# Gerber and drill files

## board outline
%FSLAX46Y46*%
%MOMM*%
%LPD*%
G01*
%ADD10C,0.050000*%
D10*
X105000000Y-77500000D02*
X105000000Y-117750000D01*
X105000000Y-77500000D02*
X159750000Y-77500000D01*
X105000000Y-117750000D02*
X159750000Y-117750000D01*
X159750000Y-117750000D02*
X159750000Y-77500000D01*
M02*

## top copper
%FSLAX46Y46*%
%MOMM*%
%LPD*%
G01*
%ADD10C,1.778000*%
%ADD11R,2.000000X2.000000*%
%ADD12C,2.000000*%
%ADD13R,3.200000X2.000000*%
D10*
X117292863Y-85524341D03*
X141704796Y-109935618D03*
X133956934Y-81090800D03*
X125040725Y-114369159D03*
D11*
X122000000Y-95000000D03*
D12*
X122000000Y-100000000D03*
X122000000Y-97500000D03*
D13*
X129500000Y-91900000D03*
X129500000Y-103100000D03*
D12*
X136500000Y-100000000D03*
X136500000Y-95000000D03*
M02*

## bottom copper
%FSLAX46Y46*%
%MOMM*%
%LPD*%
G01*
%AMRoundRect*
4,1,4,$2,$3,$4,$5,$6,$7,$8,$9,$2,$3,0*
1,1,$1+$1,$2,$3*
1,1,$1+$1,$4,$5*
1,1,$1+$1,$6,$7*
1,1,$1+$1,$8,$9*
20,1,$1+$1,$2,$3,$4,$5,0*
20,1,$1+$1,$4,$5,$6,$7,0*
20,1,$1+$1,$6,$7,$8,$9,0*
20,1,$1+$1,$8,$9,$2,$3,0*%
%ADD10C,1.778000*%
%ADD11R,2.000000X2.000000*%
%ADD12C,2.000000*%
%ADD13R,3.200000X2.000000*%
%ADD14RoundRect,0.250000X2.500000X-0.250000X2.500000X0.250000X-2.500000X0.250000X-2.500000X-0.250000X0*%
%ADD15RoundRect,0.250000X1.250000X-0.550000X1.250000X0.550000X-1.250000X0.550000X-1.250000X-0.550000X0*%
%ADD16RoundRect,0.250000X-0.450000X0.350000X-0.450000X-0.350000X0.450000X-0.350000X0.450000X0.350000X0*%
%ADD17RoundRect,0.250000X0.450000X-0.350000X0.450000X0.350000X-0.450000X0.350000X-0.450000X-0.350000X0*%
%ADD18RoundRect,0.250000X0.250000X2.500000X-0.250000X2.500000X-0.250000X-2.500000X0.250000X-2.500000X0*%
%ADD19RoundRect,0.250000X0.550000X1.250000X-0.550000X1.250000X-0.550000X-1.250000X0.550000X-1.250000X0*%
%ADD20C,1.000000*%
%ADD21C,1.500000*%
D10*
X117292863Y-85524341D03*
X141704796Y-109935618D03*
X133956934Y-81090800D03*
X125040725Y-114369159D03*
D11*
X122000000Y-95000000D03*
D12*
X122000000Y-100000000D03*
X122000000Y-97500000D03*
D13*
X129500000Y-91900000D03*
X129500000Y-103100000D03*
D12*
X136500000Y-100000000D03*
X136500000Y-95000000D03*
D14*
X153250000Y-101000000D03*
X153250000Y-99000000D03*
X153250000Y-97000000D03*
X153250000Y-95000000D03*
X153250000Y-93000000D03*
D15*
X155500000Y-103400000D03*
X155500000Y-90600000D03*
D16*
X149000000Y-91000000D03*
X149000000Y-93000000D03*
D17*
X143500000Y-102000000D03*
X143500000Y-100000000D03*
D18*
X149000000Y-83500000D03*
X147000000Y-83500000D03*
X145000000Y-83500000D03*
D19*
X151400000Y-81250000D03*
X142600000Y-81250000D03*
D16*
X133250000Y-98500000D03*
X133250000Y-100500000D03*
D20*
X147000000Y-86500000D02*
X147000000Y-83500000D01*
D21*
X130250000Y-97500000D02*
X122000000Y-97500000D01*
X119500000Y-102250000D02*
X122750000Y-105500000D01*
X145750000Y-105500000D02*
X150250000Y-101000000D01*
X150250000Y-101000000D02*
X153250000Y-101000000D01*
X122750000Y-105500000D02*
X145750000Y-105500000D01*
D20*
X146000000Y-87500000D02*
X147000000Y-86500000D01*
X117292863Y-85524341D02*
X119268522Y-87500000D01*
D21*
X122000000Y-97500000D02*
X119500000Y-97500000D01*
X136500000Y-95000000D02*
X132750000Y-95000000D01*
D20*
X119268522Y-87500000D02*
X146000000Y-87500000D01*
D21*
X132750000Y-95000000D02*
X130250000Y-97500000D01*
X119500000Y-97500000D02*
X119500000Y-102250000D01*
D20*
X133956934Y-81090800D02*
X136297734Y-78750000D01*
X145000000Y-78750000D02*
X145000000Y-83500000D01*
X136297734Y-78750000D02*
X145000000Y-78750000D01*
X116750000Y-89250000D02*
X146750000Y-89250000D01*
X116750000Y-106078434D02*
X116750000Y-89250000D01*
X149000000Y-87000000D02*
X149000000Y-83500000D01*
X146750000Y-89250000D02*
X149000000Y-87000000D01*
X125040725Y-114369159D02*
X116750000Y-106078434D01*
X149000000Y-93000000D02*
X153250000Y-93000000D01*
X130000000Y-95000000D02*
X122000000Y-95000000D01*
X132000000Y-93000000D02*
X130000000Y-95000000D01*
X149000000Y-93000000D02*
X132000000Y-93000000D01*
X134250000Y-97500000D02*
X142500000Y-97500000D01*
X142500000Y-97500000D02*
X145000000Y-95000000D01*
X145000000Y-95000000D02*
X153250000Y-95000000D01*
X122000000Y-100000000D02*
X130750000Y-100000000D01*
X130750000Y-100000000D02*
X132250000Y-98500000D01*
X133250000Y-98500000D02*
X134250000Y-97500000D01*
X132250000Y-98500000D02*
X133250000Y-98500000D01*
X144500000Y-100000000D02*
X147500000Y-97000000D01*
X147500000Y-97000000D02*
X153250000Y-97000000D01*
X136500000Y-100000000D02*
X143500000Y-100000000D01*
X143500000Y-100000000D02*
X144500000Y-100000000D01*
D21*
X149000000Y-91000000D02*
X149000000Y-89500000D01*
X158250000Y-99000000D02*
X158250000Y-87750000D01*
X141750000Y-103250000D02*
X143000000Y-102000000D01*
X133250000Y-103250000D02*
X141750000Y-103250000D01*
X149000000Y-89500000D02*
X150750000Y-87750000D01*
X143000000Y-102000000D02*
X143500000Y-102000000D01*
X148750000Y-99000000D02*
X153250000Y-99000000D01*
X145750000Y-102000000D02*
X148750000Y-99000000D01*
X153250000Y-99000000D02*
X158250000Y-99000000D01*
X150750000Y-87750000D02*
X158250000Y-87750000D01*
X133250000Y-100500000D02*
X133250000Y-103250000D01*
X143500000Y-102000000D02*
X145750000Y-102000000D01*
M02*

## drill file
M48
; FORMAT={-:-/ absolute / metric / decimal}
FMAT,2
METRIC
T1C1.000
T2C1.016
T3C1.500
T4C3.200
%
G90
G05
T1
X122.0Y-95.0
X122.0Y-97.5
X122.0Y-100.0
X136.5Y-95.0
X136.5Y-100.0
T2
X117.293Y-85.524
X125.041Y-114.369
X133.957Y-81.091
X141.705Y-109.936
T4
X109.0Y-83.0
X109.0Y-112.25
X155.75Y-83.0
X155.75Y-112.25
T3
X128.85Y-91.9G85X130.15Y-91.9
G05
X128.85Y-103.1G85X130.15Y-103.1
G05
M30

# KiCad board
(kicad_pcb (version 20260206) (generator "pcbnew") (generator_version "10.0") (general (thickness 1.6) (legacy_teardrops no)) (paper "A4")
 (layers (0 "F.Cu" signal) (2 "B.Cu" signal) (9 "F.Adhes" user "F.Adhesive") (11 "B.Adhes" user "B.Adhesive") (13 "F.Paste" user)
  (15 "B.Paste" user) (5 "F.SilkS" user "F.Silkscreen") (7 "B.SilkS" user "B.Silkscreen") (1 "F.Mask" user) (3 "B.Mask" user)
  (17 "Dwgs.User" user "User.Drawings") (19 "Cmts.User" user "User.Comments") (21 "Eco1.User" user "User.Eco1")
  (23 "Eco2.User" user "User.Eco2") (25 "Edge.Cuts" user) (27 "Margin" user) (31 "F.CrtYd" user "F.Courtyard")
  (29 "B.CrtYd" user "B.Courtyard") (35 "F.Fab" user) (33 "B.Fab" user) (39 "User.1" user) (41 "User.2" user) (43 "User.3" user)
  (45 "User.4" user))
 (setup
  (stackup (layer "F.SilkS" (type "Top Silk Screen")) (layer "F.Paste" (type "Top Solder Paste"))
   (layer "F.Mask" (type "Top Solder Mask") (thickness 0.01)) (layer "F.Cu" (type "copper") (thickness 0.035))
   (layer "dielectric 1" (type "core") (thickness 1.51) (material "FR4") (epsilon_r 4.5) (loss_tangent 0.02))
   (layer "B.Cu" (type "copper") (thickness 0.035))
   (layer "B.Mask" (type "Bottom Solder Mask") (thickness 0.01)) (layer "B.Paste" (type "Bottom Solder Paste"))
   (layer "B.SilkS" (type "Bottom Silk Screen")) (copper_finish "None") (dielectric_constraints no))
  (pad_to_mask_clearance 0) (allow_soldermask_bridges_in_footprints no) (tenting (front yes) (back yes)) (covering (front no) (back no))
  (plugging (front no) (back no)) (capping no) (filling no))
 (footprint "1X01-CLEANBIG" (layer "F.Cu") (at 117.292863 85.524341 180)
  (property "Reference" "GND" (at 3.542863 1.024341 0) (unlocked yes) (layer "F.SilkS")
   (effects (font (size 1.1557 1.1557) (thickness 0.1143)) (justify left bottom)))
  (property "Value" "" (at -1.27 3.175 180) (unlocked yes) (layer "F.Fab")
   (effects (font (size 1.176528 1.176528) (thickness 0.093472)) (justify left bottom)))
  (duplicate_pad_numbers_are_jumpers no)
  (pad "1" thru_hole circle (at 0 0 180) (size 1.778 1.778) (drill 1.016) (layers "*.Cu" "*.Mask") (remove_unused_layers no) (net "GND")
   (solder_mask_margin 0.1016) (thermal_bridge_angle 0)))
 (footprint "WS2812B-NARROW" (layer "F.Cu") (at 136.866 110.490165 -150)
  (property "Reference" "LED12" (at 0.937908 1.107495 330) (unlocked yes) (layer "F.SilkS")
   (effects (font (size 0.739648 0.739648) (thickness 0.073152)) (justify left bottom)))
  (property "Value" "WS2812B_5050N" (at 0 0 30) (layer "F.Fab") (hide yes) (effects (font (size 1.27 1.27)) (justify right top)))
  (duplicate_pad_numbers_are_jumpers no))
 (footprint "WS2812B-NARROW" (layer "F.Cu") (at 122.134 110.490165 150)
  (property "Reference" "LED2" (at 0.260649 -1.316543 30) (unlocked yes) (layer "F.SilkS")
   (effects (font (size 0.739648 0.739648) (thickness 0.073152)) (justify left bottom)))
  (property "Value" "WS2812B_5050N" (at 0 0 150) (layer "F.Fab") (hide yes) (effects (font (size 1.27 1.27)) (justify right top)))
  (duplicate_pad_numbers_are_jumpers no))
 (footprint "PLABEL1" (layer "F.Cu") (at 141.358468 108.815621 135)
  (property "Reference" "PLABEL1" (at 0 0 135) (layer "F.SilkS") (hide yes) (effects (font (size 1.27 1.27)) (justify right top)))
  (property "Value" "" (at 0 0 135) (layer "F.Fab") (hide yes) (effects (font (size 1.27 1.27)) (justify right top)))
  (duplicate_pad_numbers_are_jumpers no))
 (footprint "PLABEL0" (layer "F.Cu") (at 125.2582 111.8036 -105)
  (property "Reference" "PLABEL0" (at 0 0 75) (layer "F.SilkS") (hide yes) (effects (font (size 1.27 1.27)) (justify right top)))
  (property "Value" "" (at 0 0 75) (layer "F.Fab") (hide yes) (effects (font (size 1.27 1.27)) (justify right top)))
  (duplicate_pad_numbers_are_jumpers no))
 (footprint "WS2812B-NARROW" (layer "F.Cu") (at 142.258165 105.098 -120)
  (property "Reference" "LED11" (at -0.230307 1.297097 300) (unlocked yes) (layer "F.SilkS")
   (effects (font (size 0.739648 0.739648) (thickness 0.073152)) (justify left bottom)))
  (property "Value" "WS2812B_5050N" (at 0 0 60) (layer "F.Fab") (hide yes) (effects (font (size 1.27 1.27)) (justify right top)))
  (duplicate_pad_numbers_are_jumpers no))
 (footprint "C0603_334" (layer "F.Cu") (at 145.44739 102.00504 -15)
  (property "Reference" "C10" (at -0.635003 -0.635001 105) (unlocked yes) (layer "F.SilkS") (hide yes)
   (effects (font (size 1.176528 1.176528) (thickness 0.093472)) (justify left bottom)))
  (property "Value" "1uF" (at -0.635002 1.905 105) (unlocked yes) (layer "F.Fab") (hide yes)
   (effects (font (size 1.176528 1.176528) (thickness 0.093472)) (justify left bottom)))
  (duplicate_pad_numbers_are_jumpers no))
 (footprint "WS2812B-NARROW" (layer "F.Cu") (at 129.5 112.464 180)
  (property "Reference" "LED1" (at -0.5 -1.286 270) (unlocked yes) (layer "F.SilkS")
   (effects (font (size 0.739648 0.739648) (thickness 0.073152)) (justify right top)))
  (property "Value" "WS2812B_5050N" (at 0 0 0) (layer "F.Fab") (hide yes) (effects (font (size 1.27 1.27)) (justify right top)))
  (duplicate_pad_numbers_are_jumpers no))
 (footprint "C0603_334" (layer "F.Cu") (at 145.44739 93.45896 15)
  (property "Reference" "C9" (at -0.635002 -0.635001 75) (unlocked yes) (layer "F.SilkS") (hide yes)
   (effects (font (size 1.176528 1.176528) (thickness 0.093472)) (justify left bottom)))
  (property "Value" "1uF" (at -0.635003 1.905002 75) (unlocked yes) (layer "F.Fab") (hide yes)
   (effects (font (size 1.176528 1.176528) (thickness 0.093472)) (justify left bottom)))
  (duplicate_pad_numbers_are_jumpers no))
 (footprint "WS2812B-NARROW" (layer "F.Cu") (at 136.866 84.973835 -30)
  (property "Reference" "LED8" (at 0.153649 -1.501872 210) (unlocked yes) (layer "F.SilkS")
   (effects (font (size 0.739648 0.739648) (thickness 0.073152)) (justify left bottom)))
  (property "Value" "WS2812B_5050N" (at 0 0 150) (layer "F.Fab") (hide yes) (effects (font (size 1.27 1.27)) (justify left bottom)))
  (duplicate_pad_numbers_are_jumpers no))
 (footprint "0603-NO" (layer "F.Cu") (at 133.6 113.132 105)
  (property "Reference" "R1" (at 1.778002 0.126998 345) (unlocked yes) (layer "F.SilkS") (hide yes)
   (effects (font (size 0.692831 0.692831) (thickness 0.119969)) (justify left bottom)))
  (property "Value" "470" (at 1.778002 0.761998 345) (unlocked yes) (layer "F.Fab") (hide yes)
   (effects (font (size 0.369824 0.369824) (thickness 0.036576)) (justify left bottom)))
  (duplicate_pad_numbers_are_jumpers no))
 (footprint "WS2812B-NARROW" (layer "F.Cu") (at 122.134 84.973835 30)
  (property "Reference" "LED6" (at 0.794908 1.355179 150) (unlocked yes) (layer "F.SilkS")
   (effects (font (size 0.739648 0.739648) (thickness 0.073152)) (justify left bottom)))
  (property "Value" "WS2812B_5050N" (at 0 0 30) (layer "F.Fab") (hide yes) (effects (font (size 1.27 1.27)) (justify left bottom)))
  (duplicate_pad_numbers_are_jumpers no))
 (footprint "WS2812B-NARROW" (layer "F.Cu") (at 114.768 97.732 90)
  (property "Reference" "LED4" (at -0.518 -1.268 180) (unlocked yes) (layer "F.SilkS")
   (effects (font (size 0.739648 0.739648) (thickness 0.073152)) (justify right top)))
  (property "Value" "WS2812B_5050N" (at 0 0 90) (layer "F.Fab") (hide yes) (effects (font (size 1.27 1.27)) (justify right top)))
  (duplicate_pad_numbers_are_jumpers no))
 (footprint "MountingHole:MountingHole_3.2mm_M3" (layer "F.Cu") (at 109 83)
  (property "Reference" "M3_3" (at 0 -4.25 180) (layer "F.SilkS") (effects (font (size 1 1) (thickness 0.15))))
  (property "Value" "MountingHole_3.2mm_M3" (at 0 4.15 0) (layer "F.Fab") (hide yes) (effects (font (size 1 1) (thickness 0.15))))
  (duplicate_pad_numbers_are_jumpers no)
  (pad "" np_thru_hole circle (at 0 0) (size 3.2 3.2) (drill 3.2) (layers "*.Cu" "*.Mask")))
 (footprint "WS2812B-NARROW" (layer "F.Cu") (at 142.258165 90.366 -60)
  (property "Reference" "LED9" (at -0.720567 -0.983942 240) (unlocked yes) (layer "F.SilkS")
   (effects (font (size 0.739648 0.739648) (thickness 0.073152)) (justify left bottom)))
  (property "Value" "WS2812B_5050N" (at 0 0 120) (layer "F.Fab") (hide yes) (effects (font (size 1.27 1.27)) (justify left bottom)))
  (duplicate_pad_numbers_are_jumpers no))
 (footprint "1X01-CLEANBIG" (layer "F.Cu") (at 141.704796 109.935618 180)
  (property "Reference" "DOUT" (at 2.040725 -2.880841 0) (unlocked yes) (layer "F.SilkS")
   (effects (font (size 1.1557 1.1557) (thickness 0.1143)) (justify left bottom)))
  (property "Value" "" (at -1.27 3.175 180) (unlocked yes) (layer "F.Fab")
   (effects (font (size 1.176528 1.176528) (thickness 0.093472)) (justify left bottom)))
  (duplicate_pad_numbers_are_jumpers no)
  (pad "1" thru_hole circle (at 0 0 180) (size 1.778 1.778) (drill 1.016) (layers "*.Cu" "*.Mask") (remove_unused_layers no) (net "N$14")
   (solder_mask_margin 0.1016) (thermal_bridge_angle 0)))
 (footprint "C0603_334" (layer "F.Cu") (at 113.55261 93.45896 165)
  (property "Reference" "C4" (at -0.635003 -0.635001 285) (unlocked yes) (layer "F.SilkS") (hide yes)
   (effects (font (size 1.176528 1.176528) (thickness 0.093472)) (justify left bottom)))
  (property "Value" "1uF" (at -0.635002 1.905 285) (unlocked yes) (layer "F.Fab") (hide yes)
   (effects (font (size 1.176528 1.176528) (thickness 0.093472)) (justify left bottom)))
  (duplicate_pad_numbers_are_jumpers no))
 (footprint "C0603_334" (layer "F.Cu") (at 125.22696 81.78461 105)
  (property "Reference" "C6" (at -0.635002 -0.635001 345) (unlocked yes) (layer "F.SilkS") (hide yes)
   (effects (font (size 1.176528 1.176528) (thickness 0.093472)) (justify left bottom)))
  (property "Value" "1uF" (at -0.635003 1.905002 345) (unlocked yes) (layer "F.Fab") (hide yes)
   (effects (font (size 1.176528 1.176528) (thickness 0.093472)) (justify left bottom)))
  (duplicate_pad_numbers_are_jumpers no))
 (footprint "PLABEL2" (layer "F.Cu") (at 117.646579 86.531982 -45)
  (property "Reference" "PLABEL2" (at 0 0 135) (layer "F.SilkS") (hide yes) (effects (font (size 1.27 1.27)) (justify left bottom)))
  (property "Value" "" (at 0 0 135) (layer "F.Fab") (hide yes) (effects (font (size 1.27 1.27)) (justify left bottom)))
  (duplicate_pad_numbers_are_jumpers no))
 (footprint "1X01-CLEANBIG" (layer "F.Cu") (at 133.956934 81.0908 180)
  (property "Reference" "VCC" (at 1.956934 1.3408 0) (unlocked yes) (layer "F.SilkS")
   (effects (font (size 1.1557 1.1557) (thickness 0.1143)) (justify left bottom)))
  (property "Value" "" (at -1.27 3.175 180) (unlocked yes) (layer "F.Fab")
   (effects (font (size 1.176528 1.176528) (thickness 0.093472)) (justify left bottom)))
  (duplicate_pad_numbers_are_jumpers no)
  (pad "1" thru_hole circle (at 0 0 180) (size 1.778 1.778) (drill 1.016) (layers "*.Cu" "*.Mask") (remove_unused_layers no) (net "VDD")
   (solder_mask_margin 0.1016) (thermal_bridge_angle 0)))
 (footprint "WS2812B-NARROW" (layer "F.Cu") (at 129.5 83)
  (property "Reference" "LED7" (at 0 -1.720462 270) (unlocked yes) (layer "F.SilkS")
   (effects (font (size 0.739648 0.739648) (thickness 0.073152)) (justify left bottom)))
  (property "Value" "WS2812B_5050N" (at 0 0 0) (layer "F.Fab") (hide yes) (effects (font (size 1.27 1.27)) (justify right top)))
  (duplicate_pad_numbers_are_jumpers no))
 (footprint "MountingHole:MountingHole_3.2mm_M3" (layer "F.Cu") (at 155.75 83)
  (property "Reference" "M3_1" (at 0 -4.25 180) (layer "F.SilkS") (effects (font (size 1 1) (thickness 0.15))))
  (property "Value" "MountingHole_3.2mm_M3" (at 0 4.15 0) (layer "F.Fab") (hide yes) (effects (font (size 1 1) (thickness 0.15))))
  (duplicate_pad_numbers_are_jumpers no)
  (pad "" np_thru_hole circle (at 0 0) (size 3.2 3.2) (drill 3.2) (layers "*.Cu" "*.Mask")))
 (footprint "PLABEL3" (layer "F.Cu") (at 133.208025 81.82346 -105)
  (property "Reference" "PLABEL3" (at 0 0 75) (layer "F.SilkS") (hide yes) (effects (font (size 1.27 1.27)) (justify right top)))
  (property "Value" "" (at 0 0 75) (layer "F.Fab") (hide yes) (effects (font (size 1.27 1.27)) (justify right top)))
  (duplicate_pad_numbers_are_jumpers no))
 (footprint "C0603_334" (layer "F.Cu") (at 117.825654 109.406346 -135)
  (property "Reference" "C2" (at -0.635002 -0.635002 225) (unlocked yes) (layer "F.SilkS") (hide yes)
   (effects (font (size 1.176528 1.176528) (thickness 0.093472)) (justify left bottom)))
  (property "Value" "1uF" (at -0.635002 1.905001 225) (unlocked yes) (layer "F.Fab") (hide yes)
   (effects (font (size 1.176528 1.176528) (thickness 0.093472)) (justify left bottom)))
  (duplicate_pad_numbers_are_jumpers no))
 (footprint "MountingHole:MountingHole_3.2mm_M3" (layer "F.Cu") (at 109 112.25)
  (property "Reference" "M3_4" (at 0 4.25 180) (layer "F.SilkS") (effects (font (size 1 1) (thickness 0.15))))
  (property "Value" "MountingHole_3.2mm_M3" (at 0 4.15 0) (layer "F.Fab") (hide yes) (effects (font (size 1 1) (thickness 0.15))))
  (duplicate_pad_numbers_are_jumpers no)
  (pad "" np_thru_hole circle (at 0 0) (size 3.2 3.2) (drill 3.2) (layers "*.Cu" "*.Mask")))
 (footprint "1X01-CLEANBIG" (layer "F.Cu") (at 125.040725 114.369159 180)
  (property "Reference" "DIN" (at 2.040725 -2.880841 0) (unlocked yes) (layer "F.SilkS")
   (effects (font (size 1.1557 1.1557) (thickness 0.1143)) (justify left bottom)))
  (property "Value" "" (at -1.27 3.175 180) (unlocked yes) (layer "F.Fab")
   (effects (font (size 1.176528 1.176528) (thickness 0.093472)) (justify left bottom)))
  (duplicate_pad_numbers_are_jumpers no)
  (pad "1" thru_hole circle (at 0 0 180) (size 1.778 1.778) (drill 1.016) (layers "*.Cu" "*.Mask") (remove_unused_layers no)
   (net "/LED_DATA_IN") (solder_mask_margin 0.1016) (thermal_bridge_angle 0)))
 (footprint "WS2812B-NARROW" (layer "F.Cu") (at 116.741835 105.098 120)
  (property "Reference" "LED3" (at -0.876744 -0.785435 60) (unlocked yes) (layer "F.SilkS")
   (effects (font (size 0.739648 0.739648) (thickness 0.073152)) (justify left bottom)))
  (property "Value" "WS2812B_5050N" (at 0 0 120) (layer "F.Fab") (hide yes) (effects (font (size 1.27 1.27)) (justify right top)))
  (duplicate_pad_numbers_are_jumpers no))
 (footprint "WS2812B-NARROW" (layer "F.Cu") (at 144.232 97.732 -90)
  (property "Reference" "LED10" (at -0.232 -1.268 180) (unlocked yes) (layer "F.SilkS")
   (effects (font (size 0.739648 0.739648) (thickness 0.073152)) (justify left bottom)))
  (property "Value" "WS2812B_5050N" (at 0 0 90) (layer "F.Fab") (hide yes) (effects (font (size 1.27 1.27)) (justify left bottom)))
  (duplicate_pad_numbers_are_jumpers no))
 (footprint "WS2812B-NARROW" (layer "F.Cu") (at 116.741835 90.366 60)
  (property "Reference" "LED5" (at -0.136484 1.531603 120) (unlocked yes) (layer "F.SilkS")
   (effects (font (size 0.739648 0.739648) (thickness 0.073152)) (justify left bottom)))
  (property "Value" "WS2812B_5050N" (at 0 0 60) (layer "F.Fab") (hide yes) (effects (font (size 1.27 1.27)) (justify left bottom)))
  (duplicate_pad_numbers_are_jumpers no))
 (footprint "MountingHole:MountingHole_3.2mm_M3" (layer "F.Cu") (at 155.75 112.25)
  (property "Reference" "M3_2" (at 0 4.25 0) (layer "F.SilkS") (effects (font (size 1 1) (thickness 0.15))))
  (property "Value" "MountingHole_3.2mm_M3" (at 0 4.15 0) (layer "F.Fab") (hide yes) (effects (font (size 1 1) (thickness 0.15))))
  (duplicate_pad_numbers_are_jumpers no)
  (pad "" np_thru_hole circle (at 0 0) (size 3.2 3.2) (drill 3.2) (layers "*.Cu" "*.Mask")))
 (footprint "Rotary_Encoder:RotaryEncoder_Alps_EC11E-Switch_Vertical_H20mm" (layer "F.Cu") (at 122 95)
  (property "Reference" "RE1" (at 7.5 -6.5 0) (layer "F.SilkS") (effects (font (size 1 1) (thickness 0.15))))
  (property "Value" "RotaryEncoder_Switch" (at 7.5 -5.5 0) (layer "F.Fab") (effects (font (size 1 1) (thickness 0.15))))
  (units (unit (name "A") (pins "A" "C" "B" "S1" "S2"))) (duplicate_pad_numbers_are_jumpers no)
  (pad "A" thru_hole rect (at 0 0) (size 2 2) (drill 1) (layers "*.Cu" "*.Mask") (remove_unused_layers no) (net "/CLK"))
  (pad "B" thru_hole circle (at 0 5) (size 2 2) (drill 1) (layers "*.Cu" "*.Mask") (remove_unused_layers no) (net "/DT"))
  (pad "C" thru_hole circle (at 0 2.5) (size 2 2) (drill 1) (layers "*.Cu" "*.Mask") (remove_unused_layers no) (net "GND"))
  (pad "MP" thru_hole rect (at 7.5 -3.1) (size 3.2 2) (drill oval 2.8 1.5) (layers "*.Cu" "*.Mask") (remove_unused_layers no))
  (pad "MP" thru_hole rect (at 7.5 8.1) (size 3.2 2) (drill oval 2.8 1.5) (layers "*.Cu" "*.Mask") (remove_unused_layers no))
  (pad "S1" thru_hole circle (at 14.5 5) (size 2 2) (drill 1) (layers "*.Cu" "*.Mask") (remove_unused_layers no) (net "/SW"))
  (pad "S2" thru_hole circle (at 14.5 0) (size 2 2) (drill 1) (layers "*.Cu" "*.Mask") (remove_unused_layers no) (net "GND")))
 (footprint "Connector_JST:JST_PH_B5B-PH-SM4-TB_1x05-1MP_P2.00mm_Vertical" (layer "B.Cu") (at 153.75 97 90)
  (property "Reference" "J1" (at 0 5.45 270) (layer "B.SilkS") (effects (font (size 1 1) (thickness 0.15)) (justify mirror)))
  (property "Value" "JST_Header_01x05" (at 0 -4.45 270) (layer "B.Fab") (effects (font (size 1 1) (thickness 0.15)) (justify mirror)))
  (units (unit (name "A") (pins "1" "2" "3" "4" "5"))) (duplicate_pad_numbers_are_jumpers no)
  (pad "1" smd roundrect (at -4 -0.5 90) (size 1 5.5) (layers "B.Cu" "B.Mask" "B.Paste") (roundrect_rratio 0.25) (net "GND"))
  (pad "2" smd roundrect (at -2 -0.5 90) (size 1 5.5) (layers "B.Cu" "B.Mask" "B.Paste") (roundrect_rratio 0.25) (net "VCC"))
  (pad "3" smd roundrect (at 0 -0.5 90) (size 1 5.5) (layers "B.Cu" "B.Mask" "B.Paste") (roundrect_rratio 0.25) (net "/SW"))
  (pad "4" smd roundrect (at 2 -0.5 90) (size 1 5.5) (layers "B.Cu" "B.Mask" "B.Paste") (roundrect_rratio 0.25) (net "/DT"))
  (pad "5" smd roundrect (at 4 -0.5 90) (size 1 5.5) (layers "B.Cu" "B.Mask" "B.Paste") (roundrect_rratio 0.25) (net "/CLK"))
  (pad "MP" smd roundrect (at -6.4 1.75 90) (size 1.6 3) (layers "B.Cu" "B.Mask" "B.Paste") (roundrect_rratio 0.15625))
  (pad "MP" smd roundrect (at 6.4 1.75 90) (size 1.6 3) (layers "B.Cu" "B.Mask" "B.Paste") (roundrect_rratio 0.15625)))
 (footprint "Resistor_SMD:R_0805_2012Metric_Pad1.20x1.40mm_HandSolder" (layer "B.Cu") (at 149 92 -90)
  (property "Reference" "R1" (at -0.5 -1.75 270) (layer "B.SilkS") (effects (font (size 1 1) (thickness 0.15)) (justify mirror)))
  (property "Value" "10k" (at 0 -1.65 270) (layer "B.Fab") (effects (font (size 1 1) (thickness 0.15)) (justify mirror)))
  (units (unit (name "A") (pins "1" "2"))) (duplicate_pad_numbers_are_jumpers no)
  (pad "1" smd roundrect (at -1 0 270) (size 1.2 1.4) (layers "B.Cu" "B.Mask" "B.Paste") (roundrect_rratio 0.208333) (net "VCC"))
  (pad "2" smd roundrect (at 1 0 270) (size 1.2 1.4) (layers "B.Cu" "B.Mask" "B.Paste") (roundrect_rratio 0.208333) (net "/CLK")))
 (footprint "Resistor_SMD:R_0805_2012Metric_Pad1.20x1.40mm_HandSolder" (layer "B.Cu") (at 143.5 101 90)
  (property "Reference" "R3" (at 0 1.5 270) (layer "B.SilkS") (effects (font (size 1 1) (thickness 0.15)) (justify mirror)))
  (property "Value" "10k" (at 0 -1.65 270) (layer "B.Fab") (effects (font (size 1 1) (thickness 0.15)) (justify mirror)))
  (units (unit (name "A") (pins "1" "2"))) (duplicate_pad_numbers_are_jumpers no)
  (pad "1" smd roundrect (at -1 0 90) (size 1.2 1.4) (layers "B.Cu" "B.Mask" "B.Paste") (roundrect_rratio 0.208333) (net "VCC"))
  (pad "2" smd roundrect (at 1 0 90) (size 1.2 1.4) (layers "B.Cu" "B.Mask" "B.Paste") (roundrect_rratio 0.208333) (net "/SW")))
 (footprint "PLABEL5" (layer "B.Cu") (at 139.8124 105.4028)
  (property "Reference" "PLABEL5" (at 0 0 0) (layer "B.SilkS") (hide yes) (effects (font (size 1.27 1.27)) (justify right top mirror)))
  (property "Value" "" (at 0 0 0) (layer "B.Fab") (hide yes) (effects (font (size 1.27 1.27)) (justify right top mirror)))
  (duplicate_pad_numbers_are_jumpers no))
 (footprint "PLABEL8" (layer "B.Cu") (at 116.5714 94.8618 -90)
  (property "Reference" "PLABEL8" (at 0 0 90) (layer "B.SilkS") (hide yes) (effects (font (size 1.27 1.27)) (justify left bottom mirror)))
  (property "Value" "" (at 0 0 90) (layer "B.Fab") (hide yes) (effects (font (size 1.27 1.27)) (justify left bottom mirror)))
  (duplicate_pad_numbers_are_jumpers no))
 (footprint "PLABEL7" (layer "B.Cu") (at 130.553668 82.265816)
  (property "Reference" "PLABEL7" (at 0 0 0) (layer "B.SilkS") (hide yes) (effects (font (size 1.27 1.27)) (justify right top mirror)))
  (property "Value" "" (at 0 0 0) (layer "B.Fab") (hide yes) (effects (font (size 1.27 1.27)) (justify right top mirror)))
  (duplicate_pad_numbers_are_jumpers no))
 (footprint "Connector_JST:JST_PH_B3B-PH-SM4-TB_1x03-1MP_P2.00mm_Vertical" (layer "B.Cu") (at 147 83 180)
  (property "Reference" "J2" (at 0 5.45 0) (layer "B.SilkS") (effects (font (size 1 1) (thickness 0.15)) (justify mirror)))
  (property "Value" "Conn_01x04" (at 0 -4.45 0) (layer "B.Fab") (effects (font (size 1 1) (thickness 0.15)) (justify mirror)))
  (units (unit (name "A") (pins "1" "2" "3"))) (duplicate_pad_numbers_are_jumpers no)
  (pad "1" smd roundrect (at -2 -0.5 180) (size 1 5.5) (layers "B.Cu" "B.Mask" "B.Paste") (roundrect_rratio 0.25) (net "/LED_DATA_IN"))
  (pad "2" smd roundrect (at 0 -0.5 180) (size 1 5.5) (layers "B.Cu" "B.Mask" "B.Paste") (roundrect_rratio 0.25) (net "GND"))
  (pad "3" smd roundrect (at 2 -0.5 180) (size 1 5.5) (layers "B.Cu" "B.Mask" "B.Paste") (roundrect_rratio 0.25) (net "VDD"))
  (pad "MP" smd roundrect (at -4.4 1.75 180) (size 1.6 3) (layers "B.Cu" "B.Mask" "B.Paste") (roundrect_rratio 0.15625))
  (pad "MP" smd roundrect (at 4.4 1.75 180) (size 1.6 3) (layers "B.Cu" "B.Mask" "B.Paste") (roundrect_rratio 0.15625)))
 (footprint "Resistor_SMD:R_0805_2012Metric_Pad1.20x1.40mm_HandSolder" (layer "B.Cu") (at 133.25 99.5 -90)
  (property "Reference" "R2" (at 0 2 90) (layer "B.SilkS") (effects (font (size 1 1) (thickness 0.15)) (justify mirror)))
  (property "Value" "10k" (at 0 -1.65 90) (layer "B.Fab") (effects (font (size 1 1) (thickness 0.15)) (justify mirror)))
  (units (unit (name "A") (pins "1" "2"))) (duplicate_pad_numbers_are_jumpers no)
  (pad "1" smd roundrect (at -1 0 270) (size 1.2 1.4) (layers "B.Cu" "B.Mask" "B.Paste") (roundrect_rratio 0.208333) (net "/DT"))
  (pad "2" smd roundrect (at 1 0 270) (size 1.2 1.4) (layers "B.Cu" "B.Mask" "B.Paste") (roundrect_rratio 0.208333) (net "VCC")))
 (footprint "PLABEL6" (layer "B.Cu") (at 116.8762 87.5466)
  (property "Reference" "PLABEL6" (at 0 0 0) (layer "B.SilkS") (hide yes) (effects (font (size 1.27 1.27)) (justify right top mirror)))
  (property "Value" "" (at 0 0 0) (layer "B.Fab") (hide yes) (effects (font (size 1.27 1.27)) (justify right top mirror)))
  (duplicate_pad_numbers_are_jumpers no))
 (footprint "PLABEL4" (layer "B.Cu") (at 123.658 110.0002)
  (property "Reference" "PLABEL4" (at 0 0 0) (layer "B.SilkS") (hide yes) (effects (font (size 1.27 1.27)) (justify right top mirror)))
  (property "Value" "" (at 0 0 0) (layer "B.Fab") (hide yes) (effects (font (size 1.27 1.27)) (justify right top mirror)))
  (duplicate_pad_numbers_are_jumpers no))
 (gr_line (start 105 77.5) (end 105 117.75) (stroke (width 0.05) (type default)) (layer "Edge.Cuts"))
 (gr_line (start 105 77.5) (end 159.75 77.5) (stroke (width 0.05) (type default)) (layer "Edge.Cuts"))
 (gr_line (start 105 117.75) (end 159.75 117.75) (stroke (width 0.05) (type default)) (layer "Edge.Cuts"))
 (gr_line (start 159.75 117.75) (end 159.75 77.5) (stroke (width 0.05) (type default)) (layer "Edge.Cuts"))
 (segment (start 147 86.5) (end 147 83.5) (width 1) (layer "B.Cu") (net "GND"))
 (segment (start 130.25 97.5) (end 122 97.5) (width 1.5) (layer "B.Cu") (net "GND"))
 (segment (start 119.5 102.25) (end 122.75 105.5) (width 1.5) (layer "B.Cu") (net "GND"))
 (segment (start 145.75 105.5) (end 150.25 101) (width 1.5) (layer "B.Cu") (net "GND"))
 (segment (start 150.25 101) (end 153.25 101) (width 1.5) (layer "B.Cu") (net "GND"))
 (segment (start 122.75 105.5) (end 145.75 105.5) (width 1.5) (layer "B.Cu") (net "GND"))
 (segment (start 146 87.5) (end 147 86.5) (width 1) (layer "B.Cu") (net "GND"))
 (segment (start 117.292863 85.524341) (end 119.268522 87.5) (width 1) (layer "B.Cu") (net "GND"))
 (segment (start 122 97.5) (end 119.5 97.5) (width 1.5) (layer "B.Cu") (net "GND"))
 (segment (start 136.5 95) (end 132.75 95) (width 1.5) (layer "B.Cu") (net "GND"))
 (segment (start 119.268522 87.5) (end 146 87.5) (width 1) (layer "B.Cu") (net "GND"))
 (segment (start 132.75 95) (end 130.25 97.5) (width 1.5) (layer "B.Cu") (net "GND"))
 (segment (start 119.5 97.5) (end 119.5 102.25) (width 1.5) (layer "B.Cu") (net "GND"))
 (segment (start 133.956934 81.0908) (end 136.297734 78.75) (width 1) (layer "B.Cu") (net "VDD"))
 (segment (start 145 78.75) (end 145 83.5) (width 1) (layer "B.Cu") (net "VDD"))
 (segment (start 136.297734 78.75) (end 145 78.75) (width 1) (layer "B.Cu") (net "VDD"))
 (segment (start 116.75 89.25) (end 146.75 89.25) (width 1) (layer "B.Cu") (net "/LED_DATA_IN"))
 (segment (start 116.75 106.078434) (end 116.75 89.25) (width 1) (layer "B.Cu") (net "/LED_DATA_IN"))
 (segment (start 149 87) (end 149 83.5) (width 1) (layer "B.Cu") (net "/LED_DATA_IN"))
 (segment (start 146.75 89.25) (end 149 87) (width 1) (layer "B.Cu") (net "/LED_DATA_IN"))
 (segment (start 125.040725 114.369159) (end 116.75 106.078434) (width 1) (layer "B.Cu") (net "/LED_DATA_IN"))
 (segment (start 149 93) (end 153.25 93) (width 1) (layer "B.Cu") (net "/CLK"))
 (segment (start 130 95) (end 122 95) (width 1) (layer "B.Cu") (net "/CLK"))
 (segment (start 132 93) (end 130 95) (width 1) (layer "B.Cu") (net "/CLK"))
 (segment (start 149 93) (end 132 93) (width 1) (layer "B.Cu") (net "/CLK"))
 (segment (start 134.25 97.5) (end 142.5 97.5) (width 1) (layer "B.Cu") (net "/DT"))
 (segment (start 142.5 97.5) (end 145 95) (width 1) (layer "B.Cu") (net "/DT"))
 (segment (start 145 95) (end 153.25 95) (width 1) (layer "B.Cu") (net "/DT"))
 (segment (start 122 100) (end 130.75 100) (width 1) (layer "B.Cu") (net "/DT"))
 (segment (start 130.75 100) (end 132.25 98.5) (width 1) (layer "B.Cu") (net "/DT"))
 (segment (start 133.25 98.5) (end 134.25 97.5) (width 1) (layer "B.Cu") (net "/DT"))
 (segment (start 132.25 98.5) (end 133.25 98.5) (width 1) (layer "B.Cu") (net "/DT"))
 (segment (start 144.5 100) (end 147.5 97) (width 1) (layer "B.Cu") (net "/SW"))
 (segment (start 147.5 97) (end 153.25 97) (width 1) (layer "B.Cu") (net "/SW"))
 (segment (start 136.5 100) (end 143.5 100) (width 1) (layer "B.Cu") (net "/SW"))
 (segment (start 143.5 100) (end 144.5 100) (width 1) (layer "B.Cu") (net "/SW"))
 (segment (start 149 91) (end 149 89.5) (width 1.5) (layer "B.Cu") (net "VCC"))
 (segment (start 158.25 99) (end 158.25 87.75) (width 1.5) (layer "B.Cu") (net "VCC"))
 (segment (start 141.75 103.25) (end 143 102) (width 1.5) (layer "B.Cu") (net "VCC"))
 (segment (start 133.25 103.25) (end 141.75 103.25) (width 1.5) (layer "B.Cu") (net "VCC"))
 (segment (start 149 89.5) (end 150.75 87.75) (width 1.5) (layer "B.Cu") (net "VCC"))
 (segment (start 143 102) (end 143.5 102) (width 1.5) (layer "B.Cu") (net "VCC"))
 (segment (start 148.75 99) (end 153.25 99) (width 1.5) (layer "B.Cu") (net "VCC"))
 (segment (start 145.75 102) (end 148.75 99) (width 1.5) (layer "B.Cu") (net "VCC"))
 (segment (start 153.25 99) (end 158.25 99) (width 1.5) (layer "B.Cu") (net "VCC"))
 (segment (start 150.75 87.75) (end 158.25 87.75) (width 1.5) (layer "B.Cu") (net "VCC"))
 (segment (start 133.25 100.5) (end 133.25 103.25) (width 1.5) (layer "B.Cu") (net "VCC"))
 (segment (start 143.5 102) (end 145.75 102) (width 1.5) (layer "B.Cu") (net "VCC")))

